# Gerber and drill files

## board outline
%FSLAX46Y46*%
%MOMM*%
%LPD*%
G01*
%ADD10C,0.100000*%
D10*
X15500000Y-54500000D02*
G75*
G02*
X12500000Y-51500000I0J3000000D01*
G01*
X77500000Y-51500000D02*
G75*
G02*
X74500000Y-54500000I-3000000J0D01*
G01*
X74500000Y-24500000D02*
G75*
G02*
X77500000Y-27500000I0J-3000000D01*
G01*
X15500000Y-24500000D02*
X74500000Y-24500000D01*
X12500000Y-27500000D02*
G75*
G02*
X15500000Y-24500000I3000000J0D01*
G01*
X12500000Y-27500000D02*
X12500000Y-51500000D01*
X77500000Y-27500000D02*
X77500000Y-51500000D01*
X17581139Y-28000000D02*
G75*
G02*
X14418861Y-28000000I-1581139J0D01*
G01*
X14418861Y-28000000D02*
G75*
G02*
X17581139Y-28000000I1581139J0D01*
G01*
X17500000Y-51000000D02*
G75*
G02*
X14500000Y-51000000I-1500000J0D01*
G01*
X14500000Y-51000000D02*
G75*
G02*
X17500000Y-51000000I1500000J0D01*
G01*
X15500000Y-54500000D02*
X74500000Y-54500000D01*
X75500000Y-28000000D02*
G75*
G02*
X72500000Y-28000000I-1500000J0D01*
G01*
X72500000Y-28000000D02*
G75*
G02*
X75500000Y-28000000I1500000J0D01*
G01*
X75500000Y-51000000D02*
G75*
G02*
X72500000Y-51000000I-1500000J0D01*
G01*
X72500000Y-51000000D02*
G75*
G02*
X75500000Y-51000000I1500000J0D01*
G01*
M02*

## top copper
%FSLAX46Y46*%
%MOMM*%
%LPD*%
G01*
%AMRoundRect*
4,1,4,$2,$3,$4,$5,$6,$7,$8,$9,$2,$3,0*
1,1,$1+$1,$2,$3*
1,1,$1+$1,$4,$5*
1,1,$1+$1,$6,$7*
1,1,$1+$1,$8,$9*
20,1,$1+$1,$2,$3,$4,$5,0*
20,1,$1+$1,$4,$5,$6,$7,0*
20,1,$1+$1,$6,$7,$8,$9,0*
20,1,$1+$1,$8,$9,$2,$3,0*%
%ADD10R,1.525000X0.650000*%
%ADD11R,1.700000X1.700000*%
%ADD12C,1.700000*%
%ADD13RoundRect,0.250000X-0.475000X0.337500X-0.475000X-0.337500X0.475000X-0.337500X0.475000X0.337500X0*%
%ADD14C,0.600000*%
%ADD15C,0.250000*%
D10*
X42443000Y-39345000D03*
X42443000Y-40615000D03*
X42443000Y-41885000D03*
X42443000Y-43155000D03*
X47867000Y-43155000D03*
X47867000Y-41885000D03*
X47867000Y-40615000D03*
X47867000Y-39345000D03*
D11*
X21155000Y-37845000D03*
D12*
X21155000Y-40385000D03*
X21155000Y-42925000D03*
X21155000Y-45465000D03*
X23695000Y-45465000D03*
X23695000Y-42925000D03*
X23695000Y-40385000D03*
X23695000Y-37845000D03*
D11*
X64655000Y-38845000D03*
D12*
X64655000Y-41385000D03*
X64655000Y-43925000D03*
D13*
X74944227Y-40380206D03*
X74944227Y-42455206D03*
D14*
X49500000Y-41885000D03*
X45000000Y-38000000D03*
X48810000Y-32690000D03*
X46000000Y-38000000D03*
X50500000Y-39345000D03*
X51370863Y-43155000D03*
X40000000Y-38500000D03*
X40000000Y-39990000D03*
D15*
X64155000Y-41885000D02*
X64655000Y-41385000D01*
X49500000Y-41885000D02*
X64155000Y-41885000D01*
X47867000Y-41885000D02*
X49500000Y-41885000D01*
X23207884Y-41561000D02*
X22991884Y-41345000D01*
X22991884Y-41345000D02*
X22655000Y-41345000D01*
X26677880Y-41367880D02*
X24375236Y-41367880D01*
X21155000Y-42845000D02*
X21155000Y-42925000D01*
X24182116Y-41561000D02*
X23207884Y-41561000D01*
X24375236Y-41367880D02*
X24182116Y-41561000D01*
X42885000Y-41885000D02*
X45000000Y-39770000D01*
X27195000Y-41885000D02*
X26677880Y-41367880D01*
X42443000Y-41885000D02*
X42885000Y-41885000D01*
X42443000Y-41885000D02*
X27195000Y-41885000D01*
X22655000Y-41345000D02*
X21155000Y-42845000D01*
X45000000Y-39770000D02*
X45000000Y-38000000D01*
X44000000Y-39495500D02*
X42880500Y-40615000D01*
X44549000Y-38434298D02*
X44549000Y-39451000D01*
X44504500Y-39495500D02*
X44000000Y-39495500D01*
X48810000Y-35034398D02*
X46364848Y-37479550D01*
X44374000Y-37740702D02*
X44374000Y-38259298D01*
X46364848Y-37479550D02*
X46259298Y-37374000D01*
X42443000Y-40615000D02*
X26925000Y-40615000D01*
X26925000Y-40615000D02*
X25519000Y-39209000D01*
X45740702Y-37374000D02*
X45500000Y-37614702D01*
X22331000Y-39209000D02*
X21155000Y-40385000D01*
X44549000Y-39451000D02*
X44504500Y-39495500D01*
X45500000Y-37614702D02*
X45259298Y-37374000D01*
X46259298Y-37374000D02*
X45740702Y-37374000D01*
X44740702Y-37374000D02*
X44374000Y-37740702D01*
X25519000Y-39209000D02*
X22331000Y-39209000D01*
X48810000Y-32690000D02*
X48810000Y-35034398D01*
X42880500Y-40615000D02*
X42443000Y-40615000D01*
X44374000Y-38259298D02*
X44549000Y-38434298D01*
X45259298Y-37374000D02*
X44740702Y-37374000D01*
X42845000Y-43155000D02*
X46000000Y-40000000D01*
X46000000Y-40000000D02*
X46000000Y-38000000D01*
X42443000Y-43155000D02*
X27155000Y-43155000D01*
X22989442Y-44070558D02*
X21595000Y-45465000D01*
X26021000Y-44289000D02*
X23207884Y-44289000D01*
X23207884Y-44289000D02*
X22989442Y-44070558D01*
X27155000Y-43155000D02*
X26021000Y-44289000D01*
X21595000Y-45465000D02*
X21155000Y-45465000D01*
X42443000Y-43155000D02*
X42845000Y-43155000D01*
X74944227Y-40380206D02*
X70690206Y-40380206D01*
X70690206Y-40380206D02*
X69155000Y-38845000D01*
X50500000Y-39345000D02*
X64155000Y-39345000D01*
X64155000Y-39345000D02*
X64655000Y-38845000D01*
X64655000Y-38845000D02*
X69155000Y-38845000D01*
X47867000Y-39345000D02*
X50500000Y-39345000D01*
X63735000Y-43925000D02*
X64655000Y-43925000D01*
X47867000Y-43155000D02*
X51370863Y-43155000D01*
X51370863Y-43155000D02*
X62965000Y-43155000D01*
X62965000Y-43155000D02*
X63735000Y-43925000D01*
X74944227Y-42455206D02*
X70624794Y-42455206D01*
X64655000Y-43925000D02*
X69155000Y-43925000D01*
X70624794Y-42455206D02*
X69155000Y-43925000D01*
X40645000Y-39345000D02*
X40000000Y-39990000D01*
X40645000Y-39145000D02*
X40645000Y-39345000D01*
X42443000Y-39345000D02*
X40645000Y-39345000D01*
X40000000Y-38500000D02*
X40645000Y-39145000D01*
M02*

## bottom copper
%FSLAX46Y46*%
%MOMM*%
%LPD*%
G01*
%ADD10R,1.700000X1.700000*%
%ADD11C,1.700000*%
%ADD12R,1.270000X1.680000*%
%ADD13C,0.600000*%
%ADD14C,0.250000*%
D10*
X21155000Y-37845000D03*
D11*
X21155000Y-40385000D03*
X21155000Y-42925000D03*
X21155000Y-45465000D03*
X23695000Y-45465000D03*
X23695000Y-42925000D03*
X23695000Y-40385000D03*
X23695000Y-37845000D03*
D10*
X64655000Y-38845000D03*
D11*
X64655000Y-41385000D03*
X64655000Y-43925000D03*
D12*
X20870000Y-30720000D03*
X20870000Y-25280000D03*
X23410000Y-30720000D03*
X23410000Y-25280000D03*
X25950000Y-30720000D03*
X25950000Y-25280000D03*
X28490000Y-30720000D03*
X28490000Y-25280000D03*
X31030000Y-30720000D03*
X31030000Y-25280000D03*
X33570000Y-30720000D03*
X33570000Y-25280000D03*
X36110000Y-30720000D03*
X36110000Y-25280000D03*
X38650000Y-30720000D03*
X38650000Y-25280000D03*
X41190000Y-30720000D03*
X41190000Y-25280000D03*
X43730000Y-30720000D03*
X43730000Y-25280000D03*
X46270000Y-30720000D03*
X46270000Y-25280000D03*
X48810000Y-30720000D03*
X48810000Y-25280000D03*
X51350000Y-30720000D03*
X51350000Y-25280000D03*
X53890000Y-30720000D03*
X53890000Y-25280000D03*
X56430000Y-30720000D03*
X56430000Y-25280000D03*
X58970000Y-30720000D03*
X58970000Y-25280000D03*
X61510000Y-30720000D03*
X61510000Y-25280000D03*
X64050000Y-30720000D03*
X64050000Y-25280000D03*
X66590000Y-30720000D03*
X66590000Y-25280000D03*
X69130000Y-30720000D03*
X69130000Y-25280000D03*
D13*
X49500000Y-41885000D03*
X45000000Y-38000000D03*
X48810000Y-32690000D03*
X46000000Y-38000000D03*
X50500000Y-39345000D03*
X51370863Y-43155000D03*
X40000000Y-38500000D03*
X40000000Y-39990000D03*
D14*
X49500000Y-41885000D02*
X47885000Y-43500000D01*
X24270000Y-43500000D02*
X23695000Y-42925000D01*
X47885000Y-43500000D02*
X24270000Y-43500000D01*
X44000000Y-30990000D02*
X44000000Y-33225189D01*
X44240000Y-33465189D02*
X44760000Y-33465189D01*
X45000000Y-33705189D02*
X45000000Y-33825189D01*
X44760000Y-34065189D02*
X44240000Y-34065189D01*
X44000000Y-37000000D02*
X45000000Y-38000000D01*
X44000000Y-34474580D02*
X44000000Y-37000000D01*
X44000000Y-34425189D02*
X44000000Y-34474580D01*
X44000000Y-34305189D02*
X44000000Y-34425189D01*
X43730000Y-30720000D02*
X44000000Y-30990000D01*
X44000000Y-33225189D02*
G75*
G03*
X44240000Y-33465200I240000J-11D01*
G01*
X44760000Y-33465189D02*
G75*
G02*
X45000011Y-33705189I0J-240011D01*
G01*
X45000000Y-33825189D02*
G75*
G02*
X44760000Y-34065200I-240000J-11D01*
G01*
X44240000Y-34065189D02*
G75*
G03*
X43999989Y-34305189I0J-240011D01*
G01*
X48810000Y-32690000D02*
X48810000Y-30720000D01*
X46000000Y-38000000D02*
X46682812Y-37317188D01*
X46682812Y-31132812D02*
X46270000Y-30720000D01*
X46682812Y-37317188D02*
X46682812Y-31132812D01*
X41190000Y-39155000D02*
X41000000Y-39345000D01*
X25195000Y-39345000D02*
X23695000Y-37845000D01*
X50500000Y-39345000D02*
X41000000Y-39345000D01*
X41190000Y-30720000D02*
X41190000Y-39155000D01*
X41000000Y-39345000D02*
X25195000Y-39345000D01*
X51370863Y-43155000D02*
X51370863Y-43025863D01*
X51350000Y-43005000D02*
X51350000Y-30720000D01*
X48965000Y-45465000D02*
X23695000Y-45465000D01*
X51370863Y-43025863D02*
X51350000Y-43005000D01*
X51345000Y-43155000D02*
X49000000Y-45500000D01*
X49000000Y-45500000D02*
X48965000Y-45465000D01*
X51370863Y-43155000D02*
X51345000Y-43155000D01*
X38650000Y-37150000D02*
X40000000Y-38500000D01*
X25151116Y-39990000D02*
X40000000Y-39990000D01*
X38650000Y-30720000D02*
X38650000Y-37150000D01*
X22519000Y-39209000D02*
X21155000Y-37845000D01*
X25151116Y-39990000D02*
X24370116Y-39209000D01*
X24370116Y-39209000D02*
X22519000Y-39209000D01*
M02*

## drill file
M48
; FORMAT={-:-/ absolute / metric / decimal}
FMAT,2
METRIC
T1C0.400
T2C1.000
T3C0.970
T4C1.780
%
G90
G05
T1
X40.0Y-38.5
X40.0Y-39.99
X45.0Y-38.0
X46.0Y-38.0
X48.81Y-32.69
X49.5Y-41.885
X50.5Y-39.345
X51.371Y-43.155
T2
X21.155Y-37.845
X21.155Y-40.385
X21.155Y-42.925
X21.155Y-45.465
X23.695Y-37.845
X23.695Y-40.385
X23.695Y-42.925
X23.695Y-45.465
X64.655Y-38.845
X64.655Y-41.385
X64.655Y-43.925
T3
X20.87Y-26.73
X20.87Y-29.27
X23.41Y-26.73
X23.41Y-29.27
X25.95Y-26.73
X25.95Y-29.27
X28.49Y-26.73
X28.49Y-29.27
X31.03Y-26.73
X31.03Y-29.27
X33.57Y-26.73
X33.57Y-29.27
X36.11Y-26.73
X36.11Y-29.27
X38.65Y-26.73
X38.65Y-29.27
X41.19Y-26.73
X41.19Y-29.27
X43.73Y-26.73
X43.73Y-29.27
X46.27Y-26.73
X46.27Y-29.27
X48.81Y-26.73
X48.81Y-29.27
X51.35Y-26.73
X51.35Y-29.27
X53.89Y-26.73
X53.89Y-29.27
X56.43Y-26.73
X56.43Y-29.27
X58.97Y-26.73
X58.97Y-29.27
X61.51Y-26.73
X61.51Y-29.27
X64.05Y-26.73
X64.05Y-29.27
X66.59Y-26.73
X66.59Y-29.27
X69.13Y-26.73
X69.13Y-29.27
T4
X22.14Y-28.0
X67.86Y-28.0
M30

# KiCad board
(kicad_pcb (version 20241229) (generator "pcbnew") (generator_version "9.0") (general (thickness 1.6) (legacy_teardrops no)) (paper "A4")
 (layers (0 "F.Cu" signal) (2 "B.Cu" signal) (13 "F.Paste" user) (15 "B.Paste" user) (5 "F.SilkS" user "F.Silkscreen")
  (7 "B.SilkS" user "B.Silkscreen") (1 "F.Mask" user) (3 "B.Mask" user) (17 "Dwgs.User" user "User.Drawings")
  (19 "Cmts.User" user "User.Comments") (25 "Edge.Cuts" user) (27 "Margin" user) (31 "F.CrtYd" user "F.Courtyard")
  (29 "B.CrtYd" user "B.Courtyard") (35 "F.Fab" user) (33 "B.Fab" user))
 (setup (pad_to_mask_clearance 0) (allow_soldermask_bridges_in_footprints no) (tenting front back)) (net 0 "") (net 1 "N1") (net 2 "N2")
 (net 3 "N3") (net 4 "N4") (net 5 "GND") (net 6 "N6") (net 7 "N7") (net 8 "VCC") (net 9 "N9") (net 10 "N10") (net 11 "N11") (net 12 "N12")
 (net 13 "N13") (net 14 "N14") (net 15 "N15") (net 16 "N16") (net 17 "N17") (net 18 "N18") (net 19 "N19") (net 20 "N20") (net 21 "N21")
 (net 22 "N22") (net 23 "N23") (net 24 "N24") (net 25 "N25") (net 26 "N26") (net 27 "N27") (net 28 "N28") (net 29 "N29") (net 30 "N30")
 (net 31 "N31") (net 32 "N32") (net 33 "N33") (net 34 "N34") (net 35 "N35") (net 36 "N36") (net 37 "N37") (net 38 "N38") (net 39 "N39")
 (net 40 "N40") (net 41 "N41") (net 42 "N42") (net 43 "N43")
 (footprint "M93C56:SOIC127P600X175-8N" (layer "F.Cu") (at 45.155 41.25)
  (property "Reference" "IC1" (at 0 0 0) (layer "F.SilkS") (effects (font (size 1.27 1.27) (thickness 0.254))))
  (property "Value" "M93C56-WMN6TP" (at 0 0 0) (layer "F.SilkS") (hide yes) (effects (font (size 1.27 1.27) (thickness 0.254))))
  (pad "1" smd rect (at -2.712 -1.905 90) (size 0.65 1.525) (layers "F.Cu" "F.Mask" "F.Paste") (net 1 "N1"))
  (pad "2" smd rect (at -2.712 -0.635 90) (size 0.65 1.525) (layers "F.Cu" "F.Mask" "F.Paste") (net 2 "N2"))
  (pad "3" smd rect (at -2.712 0.635 90) (size 0.65 1.525) (layers "F.Cu" "F.Mask" "F.Paste") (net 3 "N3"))
  (pad "4" smd rect (at -2.712 1.905 90) (size 0.65 1.525) (layers "F.Cu" "F.Mask" "F.Paste") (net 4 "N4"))
  (pad "5" smd rect (at 2.712 1.905 90) (size 0.65 1.525) (layers "F.Cu" "F.Mask" "F.Paste") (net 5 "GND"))
  (pad "6" smd rect (at 2.712 0.635 90) (size 0.65 1.525) (layers "F.Cu" "F.Mask" "F.Paste") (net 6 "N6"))
  (pad "7" smd rect (at 2.712 -0.635 90) (size 0.65 1.525) (layers "F.Cu" "F.Mask" "F.Paste") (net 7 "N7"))
  (pad "8" smd rect (at 2.712 -1.905 90) (size 0.65 1.525) (layers "F.Cu" "F.Mask" "F.Paste") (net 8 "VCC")))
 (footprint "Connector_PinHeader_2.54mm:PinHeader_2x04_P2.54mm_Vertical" (layer "F.Cu") (at 21.155 37.845)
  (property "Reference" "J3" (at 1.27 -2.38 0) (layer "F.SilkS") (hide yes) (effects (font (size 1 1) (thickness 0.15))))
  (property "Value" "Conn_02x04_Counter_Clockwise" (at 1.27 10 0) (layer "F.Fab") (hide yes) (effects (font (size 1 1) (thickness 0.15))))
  (pad "1" thru_hole rect (at 0 0) (size 1.7 1.7) (drill 1) (layers "*.Cu" "*.Mask") (remove_unused_layers no) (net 1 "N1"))
  (pad "2" thru_hole circle (at 0 2.54) (size 1.7 1.7) (drill 1) (layers "*.Cu" "*.Mask") (remove_unused_layers no) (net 2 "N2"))
  (pad "3" thru_hole circle (at 0 5.08) (size 1.7 1.7) (drill 1) (layers "*.Cu" "*.Mask") (remove_unused_layers no) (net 3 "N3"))
  (pad "4" thru_hole circle (at 0 7.62) (size 1.7 1.7) (drill 1) (layers "*.Cu" "*.Mask") (remove_unused_layers no) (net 4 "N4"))
  (pad "5" thru_hole circle (at 2.54 7.62) (size 1.7 1.7) (drill 1) (layers "*.Cu" "*.Mask") (remove_unused_layers no) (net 5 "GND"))
  (pad "6" thru_hole circle (at 2.54 5.08) (size 1.7 1.7) (drill 1) (layers "*.Cu" "*.Mask") (remove_unused_layers no) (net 6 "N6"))
  (pad "7" thru_hole circle (at 2.54 2.54) (size 1.7 1.7) (drill 1) (layers "*.Cu" "*.Mask") (remove_unused_layers no) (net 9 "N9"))
  (pad "8" thru_hole circle (at 2.54 0) (size 1.7 1.7) (drill 1) (layers "*.Cu" "*.Mask") (remove_unused_layers no) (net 8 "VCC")))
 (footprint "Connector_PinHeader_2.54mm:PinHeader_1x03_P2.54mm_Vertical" (layer "F.Cu") (at 64.655 38.845)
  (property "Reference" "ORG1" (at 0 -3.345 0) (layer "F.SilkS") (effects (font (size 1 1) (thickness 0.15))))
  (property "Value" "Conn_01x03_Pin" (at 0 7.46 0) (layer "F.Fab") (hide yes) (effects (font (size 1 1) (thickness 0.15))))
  (pad "1" thru_hole rect (at 0 0) (size 1.7 1.7) (drill 1) (layers "*.Cu" "*.Mask") (remove_unused_layers no) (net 8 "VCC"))
  (pad "2" thru_hole circle (at 0 2.54) (size 1.7 1.7) (drill 1) (layers "*.Cu" "*.Mask") (remove_unused_layers no) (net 6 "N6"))
  (pad "3" thru_hole circle (at 0 5.08) (size 1.7 1.7) (drill 1) (layers "*.Cu" "*.Mask") (remove_unused_layers no) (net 5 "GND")))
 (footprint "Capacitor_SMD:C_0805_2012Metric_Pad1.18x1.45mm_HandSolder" (layer "F.Cu") (at 74.944227 41.417706 -90)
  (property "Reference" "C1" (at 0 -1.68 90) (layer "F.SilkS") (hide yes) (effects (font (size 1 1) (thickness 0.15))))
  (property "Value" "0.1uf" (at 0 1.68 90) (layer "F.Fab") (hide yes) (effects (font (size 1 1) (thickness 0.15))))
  (pad "1" smd roundrect (at -1.0375 0 270) (size 1.175 1.45) (layers "F.Cu" "F.Mask" "F.Paste") (roundrect_rratio 0.212766) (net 8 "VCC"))
  (pad "2" smd roundrect (at 1.0375 0 270) (size 1.175 1.45) (layers "F.Cu" "F.Mask" "F.Paste") (roundrect_rratio 0.212766) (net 5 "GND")))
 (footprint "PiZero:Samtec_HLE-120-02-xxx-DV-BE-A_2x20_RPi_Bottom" (layer "B.Cu") (at 45 28)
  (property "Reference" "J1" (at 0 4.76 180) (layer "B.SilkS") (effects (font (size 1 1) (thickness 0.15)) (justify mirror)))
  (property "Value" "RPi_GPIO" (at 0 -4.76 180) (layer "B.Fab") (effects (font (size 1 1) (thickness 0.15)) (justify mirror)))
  (pad "" np_thru_hole circle (at -24.13 -1.27) (size 0.97 0.97) (drill 0.97) (layers "*.Cu" "*.Mask"))
  (pad "" np_thru_hole circle (at -24.13 1.27) (size 0.97 0.97) (drill 0.97) (layers "*.Cu" "*.Mask"))
  (pad "" np_thru_hole circle (at -22.86 0) (size 1.78 1.78) (drill 1.78) (layers "*.Cu" "*.Mask"))
  (pad "" np_thru_hole circle (at -21.59 -1.27) (size 0.97 0.97) (drill 0.97) (layers "*.Cu" "*.Mask"))
  (pad "" np_thru_hole circle (at -21.59 1.27) (size 0.97 0.97) (drill 0.97) (layers "*.Cu" "*.Mask"))
  (pad "" np_thru_hole circle (at -19.05 -1.27) (size 0.97 0.97) (drill 0.97) (layers "*.Cu" "*.Mask"))
  (pad "" np_thru_hole circle (at -19.05 1.27) (size 0.97 0.97) (drill 0.97) (layers "*.Cu" "*.Mask"))
  (pad "" np_thru_hole circle (at -16.51 -1.27) (size 0.97 0.97) (drill 0.97) (layers "*.Cu" "*.Mask"))
  (pad "" np_thru_hole circle (at -16.51 1.27) (size 0.97 0.97) (drill 0.97) (layers "*.Cu" "*.Mask"))
  (pad "" np_thru_hole circle (at -13.97 -1.27) (size 0.97 0.97) (drill 0.97) (layers "*.Cu" "*.Mask"))
  (pad "" np_thru_hole circle (at -13.97 1.27) (size 0.97 0.97) (drill 0.97) (layers "*.Cu" "*.Mask"))
  (pad "" np_thru_hole circle (at -11.43 -1.27) (size 0.97 0.97) (drill 0.97) (layers "*.Cu" "*.Mask"))
  (pad "" np_thru_hole circle (at -11.43 1.27) (size 0.97 0.97) (drill 0.97) (layers "*.Cu" "*.Mask"))
  (pad "" np_thru_hole circle (at -8.89 -1.27) (size 0.97 0.97) (drill 0.97) (layers "*.Cu" "*.Mask"))
  (pad "" np_thru_hole circle (at -8.89 1.27) (size 0.97 0.97) (drill 0.97) (layers "*.Cu" "*.Mask"))
  (pad "" np_thru_hole circle (at -6.35 -1.27) (size 0.97 0.97) (drill 0.97) (layers "*.Cu" "*.Mask"))
  (pad "" np_thru_hole circle (at -6.35 1.27) (size 0.97 0.97) (drill 0.97) (layers "*.Cu" "*.Mask"))
  (pad "" np_thru_hole circle (at -3.81 -1.27) (size 0.97 0.97) (drill 0.97) (layers "*.Cu" "*.Mask"))
  (pad "" np_thru_hole circle (at -3.81 1.27) (size 0.97 0.97) (drill 0.97) (layers "*.Cu" "*.Mask"))
  (pad "" np_thru_hole circle (at -1.27 -1.27) (size 0.97 0.97) (drill 0.97) (layers "*.Cu" "*.Mask"))
  (pad "" np_thru_hole circle (at -1.27 1.27) (size 0.97 0.97) (drill 0.97) (layers "*.Cu" "*.Mask"))
  (pad "" np_thru_hole circle (at 1.27 -1.27) (size 0.97 0.97) (drill 0.97) (layers "*.Cu" "*.Mask"))
  (pad "" np_thru_hole circle (at 1.27 1.27) (size 0.97 0.97) (drill 0.97) (layers "*.Cu" "*.Mask"))
  (pad "" np_thru_hole circle (at 3.81 -1.27) (size 0.97 0.97) (drill 0.97) (layers "*.Cu" "*.Mask"))
  (pad "" np_thru_hole circle (at 3.81 1.27) (size 0.97 0.97) (drill 0.97) (layers "*.Cu" "*.Mask"))
  (pad "" np_thru_hole circle (at 6.35 -1.27) (size 0.97 0.97) (drill 0.97) (layers "*.Cu" "*.Mask"))
  (pad "" np_thru_hole circle (at 6.35 1.27) (size 0.97 0.97) (drill 0.97) (layers "*.Cu" "*.Mask"))
  (pad "" np_thru_hole circle (at 8.89 -1.27) (size 0.97 0.97) (drill 0.97) (layers "*.Cu" "*.Mask"))
  (pad "" np_thru_hole circle (at 8.89 1.27) (size 0.97 0.97) (drill 0.97) (layers "*.Cu" "*.Mask"))
  (pad "" np_thru_hole circle (at 11.43 -1.27) (size 0.97 0.97) (drill 0.97) (layers "*.Cu" "*.Mask"))
  (pad "" np_thru_hole circle (at 11.43 1.27) (size 0.97 0.97) (drill 0.97) (layers "*.Cu" "*.Mask"))
  (pad "" np_thru_hole circle (at 13.97 -1.27) (size 0.97 0.97) (drill 0.97) (layers "*.Cu" "*.Mask"))
  (pad "" np_thru_hole circle (at 13.97 1.27) (size 0.97 0.97) (drill 0.97) (layers "*.Cu" "*.Mask"))
  (pad "" np_thru_hole circle (at 16.51 -1.27) (size 0.97 0.97) (drill 0.97) (layers "*.Cu" "*.Mask"))
  (pad "" np_thru_hole circle (at 16.51 1.27) (size 0.97 0.97) (drill 0.97) (layers "*.Cu" "*.Mask"))
  (pad "" np_thru_hole circle (at 19.05 -1.27) (size 0.97 0.97) (drill 0.97) (layers "*.Cu" "*.Mask"))
  (pad "" np_thru_hole circle (at 19.05 1.27) (size 0.97 0.97) (drill 0.97) (layers "*.Cu" "*.Mask"))
  (pad "" np_thru_hole circle (at 21.59 -1.27) (size 0.97 0.97) (drill 0.97) (layers "*.Cu" "*.Mask"))
  (pad "" np_thru_hole circle (at 21.59 1.27) (size 0.97 0.97) (drill 0.97) (layers "*.Cu" "*.Mask"))
  (pad "" np_thru_hole circle (at 22.86 0) (size 1.78 1.78) (drill 1.78) (layers "*.Cu" "*.Mask"))
  (pad "" np_thru_hole circle (at 24.13 -1.27) (size 0.97 0.97) (drill 0.97) (layers "*.Cu" "*.Mask"))
  (pad "" np_thru_hole circle (at 24.13 1.27) (size 0.97 0.97) (drill 0.97) (layers "*.Cu" "*.Mask"))
  (pad "1" smd rect (at -24.13 2.72) (size 1.27 1.68) (layers "B.Cu" "B.Mask" "B.Paste") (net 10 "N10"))
  (pad "2" smd rect (at -24.13 -2.72) (size 1.27 1.68) (layers "B.Cu" "B.Mask" "B.Paste") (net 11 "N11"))
  (pad "3" smd rect (at -21.59 2.72) (size 1.27 1.68) (layers "B.Cu" "B.Mask" "B.Paste") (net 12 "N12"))
  (pad "4" smd rect (at -21.59 -2.72) (size 1.27 1.68) (layers "B.Cu" "B.Mask" "B.Paste") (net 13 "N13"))
  (pad "5" smd rect (at -19.05 2.72) (size 1.27 1.68) (layers "B.Cu" "B.Mask" "B.Paste") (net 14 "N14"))
  (pad "6" smd rect (at -19.05 -2.72) (size 1.27 1.68) (layers "B.Cu" "B.Mask" "B.Paste") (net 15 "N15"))
  (pad "7" smd rect (at -16.51 2.72) (size 1.27 1.68) (layers "B.Cu" "B.Mask" "B.Paste") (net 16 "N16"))
  (pad "8" smd rect (at -16.51 -2.72) (size 1.27 1.68) (layers "B.Cu" "B.Mask" "B.Paste") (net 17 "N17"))
  (pad "9" smd rect (at -13.97 2.72) (size 1.27 1.68) (layers "B.Cu" "B.Mask" "B.Paste") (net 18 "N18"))
  (pad "10" smd rect (at -13.97 -2.72) (size 1.27 1.68) (layers "B.Cu" "B.Mask" "B.Paste") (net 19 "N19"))
  (pad "11" smd rect (at -11.43 2.72) (size 1.27 1.68) (layers "B.Cu" "B.Mask" "B.Paste") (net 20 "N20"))
  (pad "12" smd rect (at -11.43 -2.72) (size 1.27 1.68) (layers "B.Cu" "B.Mask" "B.Paste") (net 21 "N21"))
  (pad "13" smd rect (at -8.89 2.72) (size 1.27 1.68) (layers "B.Cu" "B.Mask" "B.Paste") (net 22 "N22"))
  (pad "14" smd rect (at -8.89 -2.72) (size 1.27 1.68) (layers "B.Cu" "B.Mask" "B.Paste") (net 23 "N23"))
  (pad "15" smd rect (at -6.35 2.72) (size 1.27 1.68) (layers "B.Cu" "B.Mask" "B.Paste") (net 1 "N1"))
  (pad "16" smd rect (at -6.35 -2.72) (size 1.27 1.68) (layers "B.Cu" "B.Mask" "B.Paste") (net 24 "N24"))
  (pad "17" smd rect (at -3.81 2.72) (size 1.27 1.68) (layers "B.Cu" "B.Mask" "B.Paste") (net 8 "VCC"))
  (pad "18" smd rect (at -3.81 -2.72) (size 1.27 1.68) (layers "B.Cu" "B.Mask" "B.Paste") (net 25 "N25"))
  (pad "19" smd rect (at -1.27 2.72) (size 1.27 1.68) (layers "B.Cu" "B.Mask" "B.Paste") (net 3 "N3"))
  (pad "20" smd rect (at -1.27 -2.72) (size 1.27 1.68) (layers "B.Cu" "B.Mask" "B.Paste") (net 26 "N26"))
  (pad "21" smd rect (at 1.27 2.72) (size 1.27 1.68) (layers "B.Cu" "B.Mask" "B.Paste") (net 4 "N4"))
  (pad "22" smd rect (at 1.27 -2.72) (size 1.27 1.68) (layers "B.Cu" "B.Mask" "B.Paste") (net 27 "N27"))
  (pad "23" smd rect (at 3.81 2.72) (size 1.27 1.68) (layers "B.Cu" "B.Mask" "B.Paste") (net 2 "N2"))
  (pad "24" smd rect (at 3.81 -2.72) (size 1.27 1.68) (layers "B.Cu" "B.Mask" "B.Paste") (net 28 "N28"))
  (pad "25" smd rect (at 6.35 2.72) (size 1.27 1.68) (layers "B.Cu" "B.Mask" "B.Paste") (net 5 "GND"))
  (pad "26" smd rect (at 6.35 -2.72) (size 1.27 1.68) (layers "B.Cu" "B.Mask" "B.Paste") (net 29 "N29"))
  (pad "27" smd rect (at 8.89 2.72) (size 1.27 1.68) (layers "B.Cu" "B.Mask" "B.Paste") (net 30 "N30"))
  (pad "28" smd rect (at 8.89 -2.72) (size 1.27 1.68) (layers "B.Cu" "B.Mask" "B.Paste") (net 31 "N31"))
  (pad "29" smd rect (at 11.43 2.72) (size 1.27 1.68) (layers "B.Cu" "B.Mask" "B.Paste") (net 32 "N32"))
  (pad "30" smd rect (at 11.43 -2.72) (size 1.27 1.68) (layers "B.Cu" "B.Mask" "B.Paste") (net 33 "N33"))
  (pad "31" smd rect (at 13.97 2.72) (size 1.27 1.68) (layers "B.Cu" "B.Mask" "B.Paste") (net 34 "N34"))
  (pad "32" smd rect (at 13.97 -2.72) (size 1.27 1.68) (layers "B.Cu" "B.Mask" "B.Paste") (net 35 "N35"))
  (pad "33" smd rect (at 16.51 2.72) (size 1.27 1.68) (layers "B.Cu" "B.Mask" "B.Paste") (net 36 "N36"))
  (pad "34" smd rect (at 16.51 -2.72) (size 1.27 1.68) (layers "B.Cu" "B.Mask" "B.Paste") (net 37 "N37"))
  (pad "35" smd rect (at 19.05 2.72) (size 1.27 1.68) (layers "B.Cu" "B.Mask" "B.Paste") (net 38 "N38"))
  (pad "36" smd rect (at 19.05 -2.72) (size 1.27 1.68) (layers "B.Cu" "B.Mask" "B.Paste") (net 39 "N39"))
  (pad "37" smd rect (at 21.59 2.72) (size 1.27 1.68) (layers "B.Cu" "B.Mask" "B.Paste") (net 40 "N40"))
  (pad "38" smd rect (at 21.59 -2.72) (size 1.27 1.68) (layers "B.Cu" "B.Mask" "B.Paste") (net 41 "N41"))
  (pad "39" smd rect (at 24.13 2.72) (size 1.27 1.68) (layers "B.Cu" "B.Mask" "B.Paste") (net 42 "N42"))
  (pad "40" smd rect (at 24.13 -2.72) (size 1.27 1.68) (layers "B.Cu" "B.Mask" "B.Paste") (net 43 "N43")))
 (gr_arc (start 15.5 54.5) (mid 13.37868 53.62132) (end 12.5 51.5) (stroke (width 0.1) (type solid)) (layer "Edge.Cuts"))
 (gr_arc (start 77.5 51.5) (mid 76.62132 53.62132) (end 74.5 54.5) (stroke (width 0.1) (type solid)) (layer "Edge.Cuts"))
 (gr_arc (start 74.5 24.5) (mid 76.62132 25.37868) (end 77.5 27.5) (stroke (width 0.1) (type solid)) (layer "Edge.Cuts"))
 (gr_line (start 15.5 24.5) (end 74.5 24.5) (stroke (width 0.1) (type solid)) (layer "Edge.Cuts"))
 (gr_arc (start 12.5 27.5) (mid 13.37868 25.37868) (end 15.5 24.5) (stroke (width 0.1) (type solid)) (layer "Edge.Cuts"))
 (gr_line (start 12.5 27.5) (end 12.5 51.5) (stroke (width 0.1) (type solid)) (layer "Edge.Cuts"))
 (gr_line (start 77.5 27.5) (end 77.5 51.5) (stroke (width 0.1) (type solid)) (layer "Edge.Cuts"))
 (gr_circle (center 16 28) (end 17.5 28.5) (stroke (width 0.1) (type default)) (fill no) (layer "Edge.Cuts"))
 (gr_circle (center 16 51) (end 17.5 51) (stroke (width 0.1) (type default)) (fill no) (layer "Edge.Cuts"))
 (gr_line (start 15.5 54.5) (end 74.5 54.5) (stroke (width 0.1) (type solid)) (layer "Edge.Cuts"))
 (gr_circle (center 74 28) (end 75.5 28) (stroke (width 0.1) (type default)) (fill no) (layer "Edge.Cuts"))
 (gr_circle (center 74 51) (end 75.5 51) (stroke (width 0.1) (type default)) (fill no) (layer "Edge.Cuts"))
 (segment (start 64.155 41.885) (end 64.655 41.385) (width 0.25) (layer "F.Cu") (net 6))
 (segment (start 49.5 41.885) (end 64.155 41.885) (width 0.25) (layer "F.Cu") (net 6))
 (segment (start 47.867 41.885) (end 49.5 41.885) (width 0.25) (layer "F.Cu") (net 6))
 (via (at 49.5 41.885) (size 0.6) (drill 0.4) (layers "F.Cu" "B.Cu") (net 6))
 (segment (start 49.5 41.885) (end 47.885 43.5) (width 0.25) (layer "B.Cu") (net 6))
 (segment (start 24.27 43.5) (end 23.695 42.925) (width 0.25) (layer "B.Cu") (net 6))
 (segment (start 47.885 43.5) (end 24.27 43.5) (width 0.25) (layer "B.Cu") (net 6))
 (segment (start 23.207884 41.561) (end 22.991884 41.345) (width 0.25) (layer "F.Cu") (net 3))
 (segment (start 22.991884 41.345) (end 22.655 41.345) (width 0.25) (layer "F.Cu") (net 3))
 (segment (start 26.67788 41.36788) (end 24.375236 41.36788) (width 0.25) (layer "F.Cu") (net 3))
 (segment (start 21.155 42.845) (end 21.155 42.925) (width 0.25) (layer "F.Cu") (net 3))
 (segment (start 24.182116 41.561) (end 23.207884 41.561) (width 0.25) (layer "F.Cu") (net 3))
 (segment (start 24.375236 41.36788) (end 24.182116 41.561) (width 0.25) (layer "F.Cu") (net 3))
 (segment (start 42.885 41.885) (end 45 39.77) (width 0.25) (layer "F.Cu") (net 3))
 (segment (start 27.195 41.885) (end 26.67788 41.36788) (width 0.25) (layer "F.Cu") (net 3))
 (segment (start 42.443 41.885) (end 42.885 41.885) (width 0.25) (layer "F.Cu") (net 3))
 (segment (start 42.443 41.885) (end 27.195 41.885) (width 0.25) (layer "F.Cu") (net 3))
 (segment (start 22.655 41.345) (end 21.155 42.845) (width 0.25) (layer "F.Cu") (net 3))
 (segment (start 45 39.77) (end 45 38) (width 0.25) (layer "F.Cu") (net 3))
 (via (at 45 38) (size 0.6) (drill 0.4) (layers "F.Cu" "B.Cu") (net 3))
 (segment (start 44 30.99) (end 44 33.225189) (width 0.25) (layer "B.Cu") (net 3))
 (segment (start 44.24 33.465189) (end 44.76 33.465189) (width 0.25) (layer "B.Cu") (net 3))
 (segment (start 45 33.705189) (end 45 33.825189) (width 0.25) (layer "B.Cu") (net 3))
 (segment (start 44.76 34.065189) (end 44.24 34.065189) (width 0.25) (layer "B.Cu") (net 3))
 (segment (start 44 37) (end 45 38) (width 0.25) (layer "B.Cu") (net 3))
 (segment (start 44 34.47458) (end 44 37) (width 0.25) (layer "B.Cu") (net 3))
 (segment (start 44 34.425189) (end 44 34.47458) (width 0.25) (layer "B.Cu") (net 3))
 (segment (start 44 34.305189) (end 44 34.425189) (width 0.25) (layer "B.Cu") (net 3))
 (segment (start 43.73 30.72) (end 44 30.99) (width 0.25) (layer "B.Cu") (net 3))
 (arc (start 44 33.225189) (mid 44.070294 33.394895) (end 44.24 33.465189) (width 0.25) (layer "B.Cu") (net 3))
 (arc (start 44.76 33.465189) (mid 44.929706 33.535483) (end 45 33.705189) (width 0.25) (layer "B.Cu") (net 3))
 (arc (start 45 33.825189) (mid 44.929706 33.994895) (end 44.76 34.065189) (width 0.25) (layer "B.Cu") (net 3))
 (arc (start 44.24 34.065189) (mid 44.070294 34.135483) (end 44 34.305189) (width 0.25) (layer "B.Cu") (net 3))
 (segment (start 44 39.4955) (end 42.8805 40.615) (width 0.25) (layer "F.Cu") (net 2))
 (segment (start 44.549 38.434298) (end 44.549 39.451) (width 0.25) (layer "F.Cu") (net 2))
 (segment (start 44.5045 39.4955) (end 44 39.4955) (width 0.25) (layer "F.Cu") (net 2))
 (segment (start 48.81 35.034398) (end 46.364848 37.47955) (width 0.25) (layer "F.Cu") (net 2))
 (segment (start 44.374 37.740702) (end 44.374 38.259298) (width 0.25) (layer "F.Cu") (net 2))
 (segment (start 46.364848 37.47955) (end 46.259298 37.374) (width 0.25) (layer "F.Cu") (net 2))
 (segment (start 42.443 40.615) (end 26.925 40.615) (width 0.25) (layer "F.Cu") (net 2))
 (segment (start 26.925 40.615) (end 25.519 39.209) (width 0.25) (layer "F.Cu") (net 2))
 (segment (start 45.740702 37.374) (end 45.5 37.614702) (width 0.25) (layer "F.Cu") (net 2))
 (segment (start 22.331 39.209) (end 21.155 40.385) (width 0.25) (layer "F.Cu") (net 2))
 (segment (start 44.549 39.451) (end 44.5045 39.4955) (width 0.25) (layer "F.Cu") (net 2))
 (segment (start 45.5 37.614702) (end 45.259298 37.374) (width 0.25) (layer "F.Cu") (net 2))
 (segment (start 46.259298 37.374) (end 45.740702 37.374) (width 0.25) (layer "F.Cu") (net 2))
 (segment (start 44.740702 37.374) (end 44.374 37.740702) (width 0.25) (layer "F.Cu") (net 2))
 (segment (start 25.519 39.209) (end 22.331 39.209) (width 0.25) (layer "F.Cu") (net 2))
 (segment (start 48.81 32.69) (end 48.81 35.034398) (width 0.25) (layer "F.Cu") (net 2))
 (segment (start 42.8805 40.615) (end 42.443 40.615) (width 0.25) (layer "F.Cu") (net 2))
 (segment (start 44.374 38.259298) (end 44.549 38.434298) (width 0.25) (layer "F.Cu") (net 2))
 (segment (start 45.259298 37.374) (end 44.740702 37.374) (width 0.25) (layer "F.Cu") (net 2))
 (via (at 48.81 32.69) (size 0.6) (drill 0.4) (layers "F.Cu" "B.Cu") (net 2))
 (segment (start 48.81 32.69) (end 48.81 30.72) (width 0.25) (layer "B.Cu") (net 2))
 (segment (start 42.845 43.155) (end 46 40) (width 0.25) (layer "F.Cu") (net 4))
 (segment (start 46 40) (end 46 38) (width 0.25) (layer "F.Cu") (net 4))
 (segment (start 42.443 43.155) (end 27.155 43.155) (width 0.25) (layer "F.Cu") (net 4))
 (segment (start 22.989442 44.070558) (end 21.595 45.465) (width 0.25) (layer "F.Cu") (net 4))
 (segment (start 26.021 44.289) (end 23.207884 44.289) (width 0.25) (layer "F.Cu") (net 4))
 (segment (start 23.207884 44.289) (end 22.989442 44.070558) (width 0.25) (layer "F.Cu") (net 4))
 (segment (start 27.155 43.155) (end 26.021 44.289) (width 0.25) (layer "F.Cu") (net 4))
 (segment (start 21.595 45.465) (end 21.155 45.465) (width 0.25) (layer "F.Cu") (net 4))
 (segment (start 42.443 43.155) (end 42.845 43.155) (width 0.25) (layer "F.Cu") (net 4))
 (via (at 46 38) (size 0.6) (drill 0.4) (layers "F.Cu" "B.Cu") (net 4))
 (segment (start 46 38) (end 46.682812 37.317188) (width 0.25) (layer "B.Cu") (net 4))
 (segment (start 46.682812 31.132812) (end 46.27 30.72) (width 0.25) (layer "B.Cu") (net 4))
 (segment (start 46.682812 37.317188) (end 46.682812 31.132812) (width 0.25) (layer "B.Cu") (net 4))
 (segment (start 74.944227 40.380206) (end 70.690206 40.380206) (width 0.25) (layer "F.Cu") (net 8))
 (segment (start 70.690206 40.380206) (end 69.155 38.845) (width 0.25) (layer "F.Cu") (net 8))
 (segment (start 50.5 39.345) (end 64.155 39.345) (width 0.25) (layer "F.Cu") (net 8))
 (segment (start 64.155 39.345) (end 64.655 38.845) (width 0.25) (layer "F.Cu") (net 8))
 (segment (start 64.655 38.845) (end 69.155 38.845) (width 0.25) (layer "F.Cu") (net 8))
 (segment (start 47.867 39.345) (end 50.5 39.345) (width 0.25) (layer "F.Cu") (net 8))
 (via (at 50.5 39.345) (size 0.6) (drill 0.4) (layers "F.Cu" "B.Cu") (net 8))
 (segment (start 41.19 39.155) (end 41 39.345) (width 0.25) (layer "B.Cu") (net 8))
 (segment (start 25.195 39.345) (end 23.695 37.845) (width 0.25) (layer "B.Cu") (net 8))
 (segment (start 50.5 39.345) (end 41 39.345) (width 0.25) (layer "B.Cu") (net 8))
 (segment (start 41.19 30.72) (end 41.19 39.155) (width 0.25) (layer "B.Cu") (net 8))
 (segment (start 41 39.345) (end 25.195 39.345) (width 0.25) (layer "B.Cu") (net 8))
 (segment (start 63.735 43.925) (end 64.655 43.925) (width 0.25) (layer "F.Cu") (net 5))
 (segment (start 47.867 43.155) (end 51.370863 43.155) (width 0.25) (layer "F.Cu") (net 5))
 (segment (start 51.370863 43.155) (end 62.965 43.155) (width 0.25) (layer "F.Cu") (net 5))
 (segment (start 62.965 43.155) (end 63.735 43.925) (width 0.25) (layer "F.Cu") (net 5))
 (segment (start 74.944227 42.455206) (end 70.624794 42.455206) (width 0.25) (layer "F.Cu") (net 5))
 (segment (start 64.655 43.925) (end 69.155 43.925) (width 0.25) (layer "F.Cu") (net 5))
 (segment (start 70.624794 42.455206) (end 69.155 43.925) (width 0.25) (layer "F.Cu") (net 5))
 (via (at 51.370863 43.155) (size 0.6) (drill 0.4) (layers "F.Cu" "B.Cu") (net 5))
 (segment (start 51.370863 43.155) (end 51.370863 43.025863) (width 0.25) (layer "B.Cu") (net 5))
 (segment (start 51.35 43.005) (end 51.35 30.72) (width 0.25) (layer "B.Cu") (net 5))
 (segment (start 48.965 45.465) (end 23.695 45.465) (width 0.25) (layer "B.Cu") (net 5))
 (segment (start 51.370863 43.025863) (end 51.35 43.005) (width 0.25) (layer "B.Cu") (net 5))
 (segment (start 51.345 43.155) (end 49 45.5) (width 0.25) (layer "B.Cu") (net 5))
 (segment (start 49 45.5) (end 48.965 45.465) (width 0.25) (layer "B.Cu") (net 5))
 (segment (start 51.370863 43.155) (end 51.345 43.155) (width 0.25) (layer "B.Cu") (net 5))
 (segment (start 40.645 39.345) (end 40 39.99) (width 0.25) (layer "F.Cu") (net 1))
 (segment (start 40.645 39.145) (end 40.645 39.345) (width 0.25) (layer "F.Cu") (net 1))
 (segment (start 42.443 39.345) (end 40.645 39.345) (width 0.25) (layer "F.Cu") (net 1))
 (segment (start 40 38.5) (end 40.645 39.145) (width 0.25) (layer "F.Cu") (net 1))
 (via (at 40 38.5) (size 0.6) (drill 0.4) (layers "F.Cu" "B.Cu") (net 1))
 (via (at 40 39.99) (size 0.6) (drill 0.4) (layers "F.Cu" "B.Cu") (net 1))
 (segment (start 38.65 37.15) (end 40 38.5) (width 0.25) (layer "B.Cu") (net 1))
 (segment (start 25.151116 39.99) (end 40 39.99) (width 0.25) (layer "B.Cu") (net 1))
 (segment (start 38.65 30.72) (end 38.65 37.15) (width 0.25) (layer "B.Cu") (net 1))
 (segment (start 22.519 39.209) (end 21.155 37.845) (width 0.25) (layer "B.Cu") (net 1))
 (segment (start 25.151116 39.99) (end 24.370116 39.209) (width 0.25) (layer "B.Cu") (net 1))
 (segment (start 24.370116 39.209) (end 22.519 39.209) (width 0.25) (layer "B.Cu") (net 1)))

